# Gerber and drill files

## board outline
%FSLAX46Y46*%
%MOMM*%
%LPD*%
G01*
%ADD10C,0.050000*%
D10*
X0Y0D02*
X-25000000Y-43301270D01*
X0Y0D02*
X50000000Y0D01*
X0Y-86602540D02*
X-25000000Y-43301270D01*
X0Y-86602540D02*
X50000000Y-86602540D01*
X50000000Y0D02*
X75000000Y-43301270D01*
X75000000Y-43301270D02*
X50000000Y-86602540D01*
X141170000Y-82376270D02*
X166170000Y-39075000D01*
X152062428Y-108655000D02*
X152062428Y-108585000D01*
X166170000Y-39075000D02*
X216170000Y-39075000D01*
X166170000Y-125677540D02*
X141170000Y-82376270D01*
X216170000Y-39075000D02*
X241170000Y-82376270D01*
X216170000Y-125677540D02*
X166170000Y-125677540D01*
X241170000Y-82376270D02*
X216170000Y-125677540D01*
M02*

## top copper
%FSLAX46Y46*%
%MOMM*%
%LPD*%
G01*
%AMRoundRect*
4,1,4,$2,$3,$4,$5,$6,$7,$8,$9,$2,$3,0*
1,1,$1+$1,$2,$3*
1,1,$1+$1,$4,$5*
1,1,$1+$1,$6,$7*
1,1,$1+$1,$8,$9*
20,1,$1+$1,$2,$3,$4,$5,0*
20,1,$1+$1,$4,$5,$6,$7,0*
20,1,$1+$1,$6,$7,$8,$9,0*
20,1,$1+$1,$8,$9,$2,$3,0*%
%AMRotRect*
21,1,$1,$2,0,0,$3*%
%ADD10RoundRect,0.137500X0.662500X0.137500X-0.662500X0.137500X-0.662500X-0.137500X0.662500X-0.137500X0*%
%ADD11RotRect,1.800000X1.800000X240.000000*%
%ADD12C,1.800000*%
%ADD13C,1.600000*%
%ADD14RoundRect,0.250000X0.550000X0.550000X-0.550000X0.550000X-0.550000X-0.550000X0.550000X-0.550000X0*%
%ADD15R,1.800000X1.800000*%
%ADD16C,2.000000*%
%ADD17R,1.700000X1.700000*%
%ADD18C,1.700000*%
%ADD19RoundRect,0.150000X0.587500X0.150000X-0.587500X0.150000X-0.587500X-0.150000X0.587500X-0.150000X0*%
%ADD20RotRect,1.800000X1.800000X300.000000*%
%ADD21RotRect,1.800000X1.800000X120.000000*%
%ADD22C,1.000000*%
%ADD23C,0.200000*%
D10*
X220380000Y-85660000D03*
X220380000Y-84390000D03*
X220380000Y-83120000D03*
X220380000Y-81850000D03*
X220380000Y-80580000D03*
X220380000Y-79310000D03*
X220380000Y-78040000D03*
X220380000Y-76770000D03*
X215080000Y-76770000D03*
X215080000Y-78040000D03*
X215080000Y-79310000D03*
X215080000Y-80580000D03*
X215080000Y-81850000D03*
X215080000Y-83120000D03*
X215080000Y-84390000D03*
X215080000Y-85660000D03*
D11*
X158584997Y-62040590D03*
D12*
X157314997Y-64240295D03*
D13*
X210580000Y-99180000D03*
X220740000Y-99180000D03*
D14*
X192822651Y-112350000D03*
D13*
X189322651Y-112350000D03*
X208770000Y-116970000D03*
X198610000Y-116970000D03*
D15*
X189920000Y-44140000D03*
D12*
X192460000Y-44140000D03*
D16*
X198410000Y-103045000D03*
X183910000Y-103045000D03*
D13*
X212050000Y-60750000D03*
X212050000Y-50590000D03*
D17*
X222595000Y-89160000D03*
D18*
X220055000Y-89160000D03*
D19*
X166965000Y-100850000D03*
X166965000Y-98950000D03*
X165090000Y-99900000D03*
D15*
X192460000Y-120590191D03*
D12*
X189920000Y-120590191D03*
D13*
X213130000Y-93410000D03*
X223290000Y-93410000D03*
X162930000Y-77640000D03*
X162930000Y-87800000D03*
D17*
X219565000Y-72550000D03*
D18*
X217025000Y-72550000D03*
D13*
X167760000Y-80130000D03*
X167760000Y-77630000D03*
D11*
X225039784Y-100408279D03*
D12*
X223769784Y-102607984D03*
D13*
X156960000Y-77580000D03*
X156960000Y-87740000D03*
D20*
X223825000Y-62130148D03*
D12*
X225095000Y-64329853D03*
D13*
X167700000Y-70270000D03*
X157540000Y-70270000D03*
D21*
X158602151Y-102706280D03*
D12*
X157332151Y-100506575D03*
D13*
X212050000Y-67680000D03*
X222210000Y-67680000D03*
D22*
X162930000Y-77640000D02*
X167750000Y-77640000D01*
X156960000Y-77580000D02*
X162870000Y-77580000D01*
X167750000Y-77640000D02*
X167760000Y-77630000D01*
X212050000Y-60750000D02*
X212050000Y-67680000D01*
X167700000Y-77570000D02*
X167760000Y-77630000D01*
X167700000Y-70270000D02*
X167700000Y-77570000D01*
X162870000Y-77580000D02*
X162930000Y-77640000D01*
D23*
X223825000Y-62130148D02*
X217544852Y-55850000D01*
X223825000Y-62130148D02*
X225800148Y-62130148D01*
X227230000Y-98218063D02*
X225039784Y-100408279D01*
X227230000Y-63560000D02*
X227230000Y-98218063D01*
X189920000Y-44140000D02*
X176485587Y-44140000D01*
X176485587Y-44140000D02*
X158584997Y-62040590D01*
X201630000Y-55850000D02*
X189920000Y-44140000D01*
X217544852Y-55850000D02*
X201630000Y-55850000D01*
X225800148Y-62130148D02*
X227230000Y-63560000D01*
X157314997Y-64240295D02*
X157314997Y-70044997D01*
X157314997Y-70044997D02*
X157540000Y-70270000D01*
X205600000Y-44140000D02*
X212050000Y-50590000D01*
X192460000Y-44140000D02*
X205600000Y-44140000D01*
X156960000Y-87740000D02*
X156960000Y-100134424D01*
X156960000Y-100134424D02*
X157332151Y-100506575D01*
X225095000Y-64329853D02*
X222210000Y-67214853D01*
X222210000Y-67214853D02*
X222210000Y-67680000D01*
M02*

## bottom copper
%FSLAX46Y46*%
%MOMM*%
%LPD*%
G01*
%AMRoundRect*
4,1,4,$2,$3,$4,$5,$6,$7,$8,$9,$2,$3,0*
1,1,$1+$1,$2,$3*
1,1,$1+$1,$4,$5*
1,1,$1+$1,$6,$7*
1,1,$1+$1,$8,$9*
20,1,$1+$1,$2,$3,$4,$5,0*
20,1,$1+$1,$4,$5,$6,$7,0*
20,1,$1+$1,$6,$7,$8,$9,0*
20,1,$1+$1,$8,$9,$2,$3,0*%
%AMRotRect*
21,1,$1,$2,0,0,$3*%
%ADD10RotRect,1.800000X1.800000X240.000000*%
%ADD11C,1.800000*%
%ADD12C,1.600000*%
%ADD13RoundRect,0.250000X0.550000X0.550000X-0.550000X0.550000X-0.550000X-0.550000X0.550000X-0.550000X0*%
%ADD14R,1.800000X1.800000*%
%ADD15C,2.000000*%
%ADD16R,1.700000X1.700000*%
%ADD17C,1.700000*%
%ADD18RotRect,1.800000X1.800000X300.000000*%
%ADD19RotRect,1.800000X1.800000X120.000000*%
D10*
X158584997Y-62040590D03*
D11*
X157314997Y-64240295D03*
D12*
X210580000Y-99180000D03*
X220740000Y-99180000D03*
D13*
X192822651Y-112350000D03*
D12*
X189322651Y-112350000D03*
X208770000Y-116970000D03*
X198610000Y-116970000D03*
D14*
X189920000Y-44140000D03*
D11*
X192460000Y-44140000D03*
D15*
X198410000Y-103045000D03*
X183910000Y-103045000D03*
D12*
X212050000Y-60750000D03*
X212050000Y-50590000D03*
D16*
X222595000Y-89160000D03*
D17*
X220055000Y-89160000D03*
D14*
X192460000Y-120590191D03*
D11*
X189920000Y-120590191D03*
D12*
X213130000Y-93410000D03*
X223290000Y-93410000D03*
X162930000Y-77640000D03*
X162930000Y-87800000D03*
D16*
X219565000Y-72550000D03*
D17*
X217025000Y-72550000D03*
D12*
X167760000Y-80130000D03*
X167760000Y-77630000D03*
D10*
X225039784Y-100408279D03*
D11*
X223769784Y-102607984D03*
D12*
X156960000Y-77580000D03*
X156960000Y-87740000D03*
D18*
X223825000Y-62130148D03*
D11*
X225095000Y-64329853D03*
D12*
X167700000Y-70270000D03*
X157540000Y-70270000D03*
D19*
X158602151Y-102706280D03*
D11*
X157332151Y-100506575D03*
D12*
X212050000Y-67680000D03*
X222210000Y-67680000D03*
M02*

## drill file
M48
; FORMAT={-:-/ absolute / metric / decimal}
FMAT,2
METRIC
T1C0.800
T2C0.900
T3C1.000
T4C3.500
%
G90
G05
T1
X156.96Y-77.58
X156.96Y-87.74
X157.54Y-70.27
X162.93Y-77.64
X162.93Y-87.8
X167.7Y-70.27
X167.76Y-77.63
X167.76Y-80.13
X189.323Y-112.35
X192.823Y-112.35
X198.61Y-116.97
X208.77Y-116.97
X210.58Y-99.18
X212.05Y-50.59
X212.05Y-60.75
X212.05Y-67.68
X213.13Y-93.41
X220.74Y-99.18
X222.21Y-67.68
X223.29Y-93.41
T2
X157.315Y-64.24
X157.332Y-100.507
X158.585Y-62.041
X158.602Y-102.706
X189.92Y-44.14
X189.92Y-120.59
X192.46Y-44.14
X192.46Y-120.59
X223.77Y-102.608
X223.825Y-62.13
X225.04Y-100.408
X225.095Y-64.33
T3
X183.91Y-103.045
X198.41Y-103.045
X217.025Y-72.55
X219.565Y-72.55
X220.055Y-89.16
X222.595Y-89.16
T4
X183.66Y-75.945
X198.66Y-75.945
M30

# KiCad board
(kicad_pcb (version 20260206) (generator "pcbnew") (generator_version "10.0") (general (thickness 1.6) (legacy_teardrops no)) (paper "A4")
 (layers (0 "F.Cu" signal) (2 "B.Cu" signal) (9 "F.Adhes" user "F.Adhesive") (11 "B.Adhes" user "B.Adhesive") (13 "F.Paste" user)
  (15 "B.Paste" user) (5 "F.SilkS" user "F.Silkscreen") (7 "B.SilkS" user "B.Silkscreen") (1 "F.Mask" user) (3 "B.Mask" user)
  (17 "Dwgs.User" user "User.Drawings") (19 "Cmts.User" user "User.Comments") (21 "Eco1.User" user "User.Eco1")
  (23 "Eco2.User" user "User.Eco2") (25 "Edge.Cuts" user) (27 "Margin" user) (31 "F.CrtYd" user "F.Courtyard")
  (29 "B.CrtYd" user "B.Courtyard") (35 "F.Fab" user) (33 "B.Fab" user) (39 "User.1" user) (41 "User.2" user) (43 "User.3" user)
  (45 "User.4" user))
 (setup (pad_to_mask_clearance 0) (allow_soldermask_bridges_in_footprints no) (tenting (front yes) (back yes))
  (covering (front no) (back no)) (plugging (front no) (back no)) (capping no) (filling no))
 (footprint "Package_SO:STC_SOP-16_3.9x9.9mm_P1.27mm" (layer "F.Cu") (at 217.73 81.215 180)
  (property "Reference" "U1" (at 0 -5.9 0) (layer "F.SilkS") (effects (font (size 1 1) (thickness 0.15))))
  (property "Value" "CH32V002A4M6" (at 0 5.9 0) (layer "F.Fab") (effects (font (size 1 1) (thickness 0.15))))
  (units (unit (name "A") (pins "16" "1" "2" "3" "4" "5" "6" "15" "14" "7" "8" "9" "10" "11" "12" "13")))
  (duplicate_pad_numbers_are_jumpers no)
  (pad "1" smd roundrect (at -2.65 -4.445 180) (size 1.6 0.55) (layers "F.Cu" "F.Mask" "F.Paste") (roundrect_rratio 0.25)
   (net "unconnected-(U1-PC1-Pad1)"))
  (pad "2" smd roundrect (at -2.65 -3.175 180) (size 1.6 0.55) (layers "F.Cu" "F.Mask" "F.Paste") (roundrect_rratio 0.25)
   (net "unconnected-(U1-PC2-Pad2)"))
  (pad "3" smd roundrect (at -2.65 -1.905 180) (size 1.6 0.55) (layers "F.Cu" "F.Mask" "F.Paste") (roundrect_rratio 0.25) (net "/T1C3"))
  (pad "4" smd roundrect (at -2.65 -0.635 180) (size 1.6 0.55) (layers "F.Cu" "F.Mask" "F.Paste") (roundrect_rratio 0.25)
   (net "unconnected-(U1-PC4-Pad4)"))
  (pad "5" smd roundrect (at -2.65 0.635 180) (size 1.6 0.55) (layers "F.Cu" "F.Mask" "F.Paste") (roundrect_rratio 0.25)
   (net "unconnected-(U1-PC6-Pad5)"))
  (pad "6" smd roundrect (at -2.65 1.905 180) (size 1.6 0.55) (layers "F.Cu" "F.Mask" "F.Paste") (roundrect_rratio 0.25)
   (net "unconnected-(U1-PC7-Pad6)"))
  (pad "7" smd roundrect (at -2.65 3.175 180) (size 1.6 0.55) (layers "F.Cu" "F.Mask" "F.Paste") (roundrect_rratio 0.25) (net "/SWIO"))
  (pad "8" smd roundrect (at -2.65 4.445 180) (size 1.6 0.55) (layers "F.Cu" "F.Mask" "F.Paste") (roundrect_rratio 0.25)
   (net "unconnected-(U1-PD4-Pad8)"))
  (pad "9" smd roundrect (at 2.65 4.445 180) (size 1.6 0.55) (layers "F.Cu" "F.Mask" "F.Paste") (roundrect_rratio 0.25)
   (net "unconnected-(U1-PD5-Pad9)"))
  (pad "10" smd roundrect (at 2.65 3.175 180) (size 1.6 0.55) (layers "F.Cu" "F.Mask" "F.Paste") (roundrect_rratio 0.25)
   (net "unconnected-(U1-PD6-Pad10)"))
  (pad "11" smd roundrect (at 2.65 1.905 180) (size 1.6 0.55) (layers "F.Cu" "F.Mask" "F.Paste") (roundrect_rratio 0.25)
   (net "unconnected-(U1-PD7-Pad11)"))
  (pad "12" smd roundrect (at 2.65 0.635 180) (size 1.6 0.55) (layers "F.Cu" "F.Mask" "F.Paste") (roundrect_rratio 0.25)
   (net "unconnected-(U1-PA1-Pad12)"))
  (pad "13" smd roundrect (at 2.65 -0.635 180) (size 1.6 0.55) (layers "F.Cu" "F.Mask" "F.Paste") (roundrect_rratio 0.25)
   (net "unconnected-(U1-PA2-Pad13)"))
  (pad "14" smd roundrect (at 2.65 -1.905 180) (size 1.6 0.55) (layers "F.Cu" "F.Mask" "F.Paste") (roundrect_rratio 0.25) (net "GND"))
  (pad "15" smd roundrect (at 2.65 -3.175 180) (size 1.6 0.55) (layers "F.Cu" "F.Mask" "F.Paste") (roundrect_rratio 0.25) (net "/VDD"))
  (pad "16" smd roundrect (at 2.65 -4.445 180) (size 1.6 0.55) (layers "F.Cu" "F.Mask" "F.Paste") (roundrect_rratio 0.25)
   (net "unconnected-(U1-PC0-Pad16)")))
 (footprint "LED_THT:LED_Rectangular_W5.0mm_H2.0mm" (layer "F.Cu") (at 158.584997 62.04059 -120)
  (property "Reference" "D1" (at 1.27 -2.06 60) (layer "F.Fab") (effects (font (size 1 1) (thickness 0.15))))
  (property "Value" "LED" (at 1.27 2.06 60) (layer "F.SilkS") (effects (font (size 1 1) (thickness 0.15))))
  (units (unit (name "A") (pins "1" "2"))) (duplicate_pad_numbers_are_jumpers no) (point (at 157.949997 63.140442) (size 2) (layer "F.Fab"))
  (pad "1" thru_hole rect (at 0 0 240) (size 1.8 1.8) (drill 0.9) (layers "*.Cu" "*.Mask") (remove_unused_layers no) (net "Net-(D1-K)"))
  (pad "2" thru_hole circle (at 2.54 0 240) (size 1.8 1.8) (drill 0.9) (layers "*.Cu" "*.Mask") (remove_unused_layers no) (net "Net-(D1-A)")))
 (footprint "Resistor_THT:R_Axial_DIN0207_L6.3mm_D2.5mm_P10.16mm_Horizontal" (layer "F.Cu") (at 210.58 99.18)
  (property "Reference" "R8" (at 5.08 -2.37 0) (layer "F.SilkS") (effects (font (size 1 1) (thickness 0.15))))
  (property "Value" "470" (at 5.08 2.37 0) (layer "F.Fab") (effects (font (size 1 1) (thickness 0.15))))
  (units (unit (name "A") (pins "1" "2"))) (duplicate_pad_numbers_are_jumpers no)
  (pad "1" thru_hole circle (at 0 0) (size 1.6 1.6) (drill 0.8) (layers "*.Cu" "*.Mask") (remove_unused_layers no) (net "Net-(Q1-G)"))
  (pad "2" thru_hole circle (at 10.16 0) (size 1.6 1.6) (drill 0.8) (layers "*.Cu" "*.Mask") (remove_unused_layers no) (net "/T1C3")))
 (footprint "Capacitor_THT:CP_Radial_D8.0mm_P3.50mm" (layer "F.Cu") (at 192.822651 112.35 180)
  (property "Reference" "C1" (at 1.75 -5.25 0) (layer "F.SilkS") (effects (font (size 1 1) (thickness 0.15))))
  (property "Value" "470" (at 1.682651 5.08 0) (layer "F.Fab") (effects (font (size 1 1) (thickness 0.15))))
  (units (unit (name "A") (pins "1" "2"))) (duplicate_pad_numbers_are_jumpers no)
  (pad "1" thru_hole roundrect (at 0 0 180) (size 1.6 1.6) (drill 0.8) (layers "*.Cu" "*.Mask") (remove_unused_layers no)
   (roundrect_rratio 0.15625) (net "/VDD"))
  (pad "2" thru_hole circle (at 3.5 0 180) (size 1.6 1.6) (drill 0.8) (layers "*.Cu" "*.Mask") (remove_unused_layers no) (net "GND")))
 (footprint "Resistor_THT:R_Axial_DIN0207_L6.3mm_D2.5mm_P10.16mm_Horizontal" (layer "F.Cu") (at 208.77 116.97 180)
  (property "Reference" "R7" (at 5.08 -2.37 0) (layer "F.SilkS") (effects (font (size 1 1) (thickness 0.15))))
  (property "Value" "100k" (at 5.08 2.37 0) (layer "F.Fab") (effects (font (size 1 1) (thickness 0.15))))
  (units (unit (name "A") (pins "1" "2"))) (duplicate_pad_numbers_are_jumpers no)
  (pad "1" thru_hole circle (at 0 0 180) (size 1.6 1.6) (drill 0.8) (layers "*.Cu" "*.Mask") (remove_unused_layers no) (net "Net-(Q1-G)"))
  (pad "2" thru_hole circle (at 10.16 0 180) (size 1.6 1.6) (drill 0.8) (layers "*.Cu" "*.Mask") (remove_unused_layers no) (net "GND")))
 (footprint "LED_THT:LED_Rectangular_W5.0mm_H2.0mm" (layer "F.Cu") (at 189.92 44.14)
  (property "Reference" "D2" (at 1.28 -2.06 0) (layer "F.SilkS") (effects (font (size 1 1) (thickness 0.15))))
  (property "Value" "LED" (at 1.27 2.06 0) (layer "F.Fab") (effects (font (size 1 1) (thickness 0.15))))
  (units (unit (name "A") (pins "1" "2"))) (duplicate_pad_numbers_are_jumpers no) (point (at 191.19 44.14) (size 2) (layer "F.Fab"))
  (pad "1" thru_hole rect (at 0 0) (size 1.8 1.8) (drill 0.9) (layers "*.Cu" "*.Mask") (remove_unused_layers no) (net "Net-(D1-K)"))
  (pad "2" thru_hole circle (at 2.54 0) (size 1.8 1.8) (drill 0.9) (layers "*.Cu" "*.Mask") (remove_unused_layers no) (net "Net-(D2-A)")))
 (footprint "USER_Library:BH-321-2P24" (layer "F.Cu") (at 191.16 75.945 -90)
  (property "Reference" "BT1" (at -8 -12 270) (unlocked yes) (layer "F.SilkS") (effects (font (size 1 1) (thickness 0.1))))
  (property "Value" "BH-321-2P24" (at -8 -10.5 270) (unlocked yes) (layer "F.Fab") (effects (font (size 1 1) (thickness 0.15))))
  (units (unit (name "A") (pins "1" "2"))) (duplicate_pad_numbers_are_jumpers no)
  (pad "" np_thru_hole circle (at 0 -7.5 270) (size 3.5 3.5) (drill 3.5) (layers "*.Cu" "*.Mask") (thermal_bridge_angle 90))
  (pad "" np_thru_hole circle (at 0 7.5 270) (size 3.5 3.5) (drill 3.5) (layers "*.Cu" "*.Mask") (thermal_bridge_angle 90))
  (pad "1" thru_hole circle (at 27.1 -7.25 270) (size 2 2) (drill 1) (layers "*.Cu" "*.Mask") (remove_unused_layers no) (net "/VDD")
   (thermal_bridge_angle 90))
  (pad "2" thru_hole circle (at 27.1 7.25 270) (size 2 2) (drill 1) (layers "*.Cu" "*.Mask") (remove_unused_layers no) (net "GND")
   (thermal_bridge_angle 90)))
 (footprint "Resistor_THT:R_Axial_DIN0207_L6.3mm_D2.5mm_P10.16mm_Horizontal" (layer "F.Cu") (at 212.05 60.75 90)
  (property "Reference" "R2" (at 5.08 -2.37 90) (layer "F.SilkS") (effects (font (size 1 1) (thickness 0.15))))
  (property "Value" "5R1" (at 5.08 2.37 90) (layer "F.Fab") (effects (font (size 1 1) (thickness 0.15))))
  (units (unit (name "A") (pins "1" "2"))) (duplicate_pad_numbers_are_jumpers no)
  (pad "1" thru_hole circle (at 0 0 90) (size 1.6 1.6) (drill 0.8) (layers "*.Cu" "*.Mask") (remove_unused_layers no) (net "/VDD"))
  (pad "2" thru_hole circle (at 10.16 0 90) (size 1.6 1.6) (drill 0.8) (layers "*.Cu" "*.Mask") (remove_unused_layers no) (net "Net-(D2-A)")))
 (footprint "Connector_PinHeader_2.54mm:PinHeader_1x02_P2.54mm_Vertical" (layer "F.Cu") (at 222.595 89.16 -90)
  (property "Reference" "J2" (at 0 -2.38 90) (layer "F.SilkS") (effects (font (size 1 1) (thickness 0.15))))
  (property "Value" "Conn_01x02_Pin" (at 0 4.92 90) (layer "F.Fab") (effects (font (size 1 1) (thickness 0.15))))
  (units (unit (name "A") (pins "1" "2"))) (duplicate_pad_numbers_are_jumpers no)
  (pad "1" thru_hole rect (at 0 0 270) (size 1.7 1.7) (drill 1) (layers "*.Cu" "*.Mask") (remove_unused_layers no) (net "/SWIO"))
  (pad "2" thru_hole circle (at 0 2.54 270) (size 1.7 1.7) (drill 1) (layers "*.Cu" "*.Mask") (remove_unused_layers no) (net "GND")))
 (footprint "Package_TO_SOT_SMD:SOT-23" (layer "F.Cu") (at 166.0275 99.9 180)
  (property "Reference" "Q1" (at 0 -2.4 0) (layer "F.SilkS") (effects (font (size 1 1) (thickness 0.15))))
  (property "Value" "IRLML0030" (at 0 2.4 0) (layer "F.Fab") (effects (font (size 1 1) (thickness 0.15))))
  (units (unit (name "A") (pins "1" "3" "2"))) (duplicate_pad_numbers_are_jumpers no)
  (pad "1" smd roundrect (at -0.9375 -0.95 180) (size 1.475 0.6) (layers "F.Cu" "F.Mask" "F.Paste") (roundrect_rratio 0.25)
   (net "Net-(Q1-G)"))
  (pad "2" smd roundrect (at -0.9375 0.95 180) (size 1.475 0.6) (layers "F.Cu" "F.Mask" "F.Paste") (roundrect_rratio 0.25) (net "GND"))
  (pad "3" smd roundrect (at 0.9375 0 180) (size 1.475 0.6) (layers "F.Cu" "F.Mask" "F.Paste") (roundrect_rratio 0.25) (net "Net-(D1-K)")))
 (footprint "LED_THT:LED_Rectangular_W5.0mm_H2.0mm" (layer "F.Cu") (at 192.46 120.590191 180)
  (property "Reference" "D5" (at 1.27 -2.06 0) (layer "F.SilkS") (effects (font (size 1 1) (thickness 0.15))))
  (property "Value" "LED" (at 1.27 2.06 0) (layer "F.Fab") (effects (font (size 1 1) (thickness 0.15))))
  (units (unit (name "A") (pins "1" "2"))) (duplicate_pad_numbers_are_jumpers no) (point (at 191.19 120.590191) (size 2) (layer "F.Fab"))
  (pad "1" thru_hole rect (at 0 0 180) (size 1.8 1.8) (drill 0.9) (layers "*.Cu" "*.Mask") (remove_unused_layers no) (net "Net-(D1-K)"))
  (pad "2" thru_hole circle (at 2.54 0 180) (size 1.8 1.8) (drill 0.9) (layers "*.Cu" "*.Mask") (remove_unused_layers no) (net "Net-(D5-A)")))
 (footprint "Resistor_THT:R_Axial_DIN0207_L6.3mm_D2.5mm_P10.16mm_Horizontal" (layer "F.Cu") (at 213.13 93.41)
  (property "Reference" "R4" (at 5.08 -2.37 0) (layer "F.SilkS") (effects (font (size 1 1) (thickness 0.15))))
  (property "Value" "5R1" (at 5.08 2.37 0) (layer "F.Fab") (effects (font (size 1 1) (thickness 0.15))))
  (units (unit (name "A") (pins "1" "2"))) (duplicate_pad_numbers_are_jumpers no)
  (pad "1" thru_hole circle (at 0 0) (size 1.6 1.6) (drill 0.8) (layers "*.Cu" "*.Mask") (remove_unused_layers no) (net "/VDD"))
  (pad "2" thru_hole circle (at 10.16 0) (size 1.6 1.6) (drill 0.8) (layers "*.Cu" "*.Mask") (remove_unused_layers no) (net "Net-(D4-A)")))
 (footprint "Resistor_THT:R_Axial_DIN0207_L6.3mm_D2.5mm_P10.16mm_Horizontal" (layer "F.Cu") (at 162.93 77.64 -90)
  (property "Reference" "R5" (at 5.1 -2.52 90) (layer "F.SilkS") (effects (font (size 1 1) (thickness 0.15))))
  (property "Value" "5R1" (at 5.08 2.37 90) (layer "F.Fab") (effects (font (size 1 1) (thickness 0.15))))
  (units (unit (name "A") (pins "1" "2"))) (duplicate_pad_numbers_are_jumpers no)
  (pad "1" thru_hole circle (at 0 0 270) (size 1.6 1.6) (drill 0.8) (layers "*.Cu" "*.Mask") (remove_unused_layers no) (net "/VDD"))
  (pad "2" thru_hole circle (at 10.16 0 270) (size 1.6 1.6) (drill 0.8) (layers "*.Cu" "*.Mask") (remove_unused_layers no)
   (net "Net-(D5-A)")))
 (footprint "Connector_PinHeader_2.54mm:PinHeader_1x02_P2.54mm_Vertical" (layer "F.Cu") (at 219.565 72.55 -90)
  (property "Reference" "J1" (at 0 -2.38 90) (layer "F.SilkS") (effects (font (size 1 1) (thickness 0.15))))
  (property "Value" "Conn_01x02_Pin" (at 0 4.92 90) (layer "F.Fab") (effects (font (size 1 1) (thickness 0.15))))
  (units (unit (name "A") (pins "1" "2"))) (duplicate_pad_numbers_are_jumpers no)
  (pad "1" thru_hole rect (at 0 0 270) (size 1.7 1.7) (drill 1) (layers "*.Cu" "*.Mask") (remove_unused_layers no) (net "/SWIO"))
  (pad "2" thru_hole circle (at 0 2.54 270) (size 1.7 1.7) (drill 1) (layers "*.Cu" "*.Mask") (remove_unused_layers no) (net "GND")))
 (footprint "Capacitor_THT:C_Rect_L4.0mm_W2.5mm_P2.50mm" (layer "F.Cu") (at 167.76 80.13 90)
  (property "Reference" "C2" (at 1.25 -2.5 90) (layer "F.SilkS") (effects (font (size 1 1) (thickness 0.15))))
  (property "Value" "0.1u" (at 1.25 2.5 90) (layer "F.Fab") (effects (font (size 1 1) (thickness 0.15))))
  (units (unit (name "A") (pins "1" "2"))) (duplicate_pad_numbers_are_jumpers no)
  (pad "1" thru_hole circle (at 0 0 90) (size 1.6 1.6) (drill 0.8) (layers "*.Cu" "*.Mask") (remove_unused_layers no) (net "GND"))
  (pad "2" thru_hole circle (at 2.5 0 90) (size 1.6 1.6) (drill 0.8) (layers "*.Cu" "*.Mask") (remove_unused_layers no) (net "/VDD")))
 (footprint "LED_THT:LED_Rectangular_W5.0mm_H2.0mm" (layer "F.Cu") (at 225.039784 100.408279 -120)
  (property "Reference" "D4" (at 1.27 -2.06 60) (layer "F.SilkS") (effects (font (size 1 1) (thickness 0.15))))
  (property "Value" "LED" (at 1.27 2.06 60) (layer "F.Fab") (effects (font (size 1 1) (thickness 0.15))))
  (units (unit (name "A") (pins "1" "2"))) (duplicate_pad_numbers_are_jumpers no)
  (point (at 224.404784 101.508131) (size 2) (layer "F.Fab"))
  (pad "1" thru_hole rect (at 0 0 240) (size 1.8 1.8) (drill 0.9) (layers "*.Cu" "*.Mask") (remove_unused_layers no) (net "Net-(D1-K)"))
  (pad "2" thru_hole circle (at 2.54 0 240) (size 1.8 1.8) (drill 0.9) (layers "*.Cu" "*.Mask") (remove_unused_layers no) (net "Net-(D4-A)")))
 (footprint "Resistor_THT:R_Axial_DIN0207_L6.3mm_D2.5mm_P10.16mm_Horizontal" (layer "F.Cu") (at 156.96 77.58 -90)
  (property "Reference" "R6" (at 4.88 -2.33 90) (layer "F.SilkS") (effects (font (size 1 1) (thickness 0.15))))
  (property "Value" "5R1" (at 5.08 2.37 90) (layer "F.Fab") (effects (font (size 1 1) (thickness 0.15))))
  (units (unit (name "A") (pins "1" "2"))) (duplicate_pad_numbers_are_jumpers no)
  (pad "1" thru_hole circle (at 0 0 270) (size 1.6 1.6) (drill 0.8) (layers "*.Cu" "*.Mask") (remove_unused_layers no) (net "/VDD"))
  (pad "2" thru_hole circle (at 10.16 0 270) (size 1.6 1.6) (drill 0.8) (layers "*.Cu" "*.Mask") (remove_unused_layers no)
   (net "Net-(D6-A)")))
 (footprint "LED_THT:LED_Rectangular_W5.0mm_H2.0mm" (layer "F.Cu") (at 223.825 62.130148 -60)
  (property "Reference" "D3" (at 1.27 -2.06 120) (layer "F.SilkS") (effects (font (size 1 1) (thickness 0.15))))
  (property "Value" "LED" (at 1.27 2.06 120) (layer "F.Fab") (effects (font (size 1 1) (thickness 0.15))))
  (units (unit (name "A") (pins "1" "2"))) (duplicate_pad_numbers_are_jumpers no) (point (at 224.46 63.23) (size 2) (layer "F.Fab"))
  (pad "1" thru_hole rect (at 0 0 300) (size 1.8 1.8) (drill 0.9) (layers "*.Cu" "*.Mask") (remove_unused_layers no) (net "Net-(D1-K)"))
  (pad "2" thru_hole circle (at 2.54 0 300) (size 1.8 1.8) (drill 0.9) (layers "*.Cu" "*.Mask") (remove_unused_layers no) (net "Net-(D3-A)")))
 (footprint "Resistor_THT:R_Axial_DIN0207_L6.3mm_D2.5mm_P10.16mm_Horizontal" (layer "F.Cu") (at 167.7 70.27 180)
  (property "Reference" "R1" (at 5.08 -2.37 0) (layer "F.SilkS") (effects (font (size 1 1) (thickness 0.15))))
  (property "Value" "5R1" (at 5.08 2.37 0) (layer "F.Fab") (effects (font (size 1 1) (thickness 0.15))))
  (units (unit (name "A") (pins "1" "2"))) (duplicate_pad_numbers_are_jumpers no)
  (pad "1" thru_hole circle (at 0 0 180) (size 1.6 1.6) (drill 0.8) (layers "*.Cu" "*.Mask") (remove_unused_layers no) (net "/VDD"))
  (pad "2" thru_hole circle (at 10.16 0 180) (size 1.6 1.6) (drill 0.8) (layers "*.Cu" "*.Mask") (remove_unused_layers no)
   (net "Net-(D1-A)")))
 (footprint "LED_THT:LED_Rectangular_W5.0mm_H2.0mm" (layer "F.Cu") (at 158.602151 102.70628 120)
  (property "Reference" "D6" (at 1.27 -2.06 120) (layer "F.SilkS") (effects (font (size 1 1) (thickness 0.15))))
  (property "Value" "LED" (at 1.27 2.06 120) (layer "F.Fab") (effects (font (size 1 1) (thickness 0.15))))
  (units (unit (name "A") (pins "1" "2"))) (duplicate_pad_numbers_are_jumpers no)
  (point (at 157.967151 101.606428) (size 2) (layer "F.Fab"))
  (pad "1" thru_hole rect (at 0 0 120) (size 1.8 1.8) (drill 0.9) (layers "*.Cu" "*.Mask") (remove_unused_layers no) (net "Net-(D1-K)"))
  (pad "2" thru_hole circle (at 2.54 0 120) (size 1.8 1.8) (drill 0.9) (layers "*.Cu" "*.Mask") (remove_unused_layers no) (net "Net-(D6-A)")))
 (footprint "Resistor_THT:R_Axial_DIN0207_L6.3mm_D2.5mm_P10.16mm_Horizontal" (layer "F.Cu") (at 212.05 67.68)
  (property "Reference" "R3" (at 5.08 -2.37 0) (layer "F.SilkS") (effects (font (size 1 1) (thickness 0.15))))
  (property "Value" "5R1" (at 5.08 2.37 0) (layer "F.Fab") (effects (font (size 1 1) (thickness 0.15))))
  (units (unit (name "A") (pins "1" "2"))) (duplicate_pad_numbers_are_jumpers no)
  (pad "1" thru_hole circle (at 0 0) (size 1.6 1.6) (drill 0.8) (layers "*.Cu" "*.Mask") (remove_unused_layers no) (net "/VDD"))
  (pad "2" thru_hole circle (at 10.16 0) (size 1.6 1.6) (drill 0.8) (layers "*.Cu" "*.Mask") (remove_unused_layers no) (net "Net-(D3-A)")))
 (gr_line (start 0 0) (end -25 43.30127) (stroke (width 0.05) (type solid)) (locked yes) (layer "Edge.Cuts"))
 (gr_line (start 0 0) (end 50 0) (stroke (width 0.05) (type solid)) (locked yes) (layer "Edge.Cuts"))
 (gr_line (start 0 86.60254) (end -25 43.30127) (stroke (width 0.05) (type solid)) (locked yes) (layer "Edge.Cuts"))
 (gr_line (start 0 86.60254) (end 50 86.60254) (stroke (width 0.05) (type solid)) (locked yes) (layer "Edge.Cuts"))
 (gr_line (start 50 0) (end 75 43.30127) (stroke (width 0.05) (type solid)) (locked yes) (layer "Edge.Cuts"))
 (gr_line (start 75 43.30127) (end 50 86.60254) (stroke (width 0.05) (type solid)) (locked yes) (layer "Edge.Cuts"))
 (gr_line (start 141.17 82.37627) (end 166.17 39.075) (stroke (width 0.05) (type default)) (layer "Edge.Cuts"))
 (gr_line (start 152.062428 108.655) (end 152.062428 108.585) (stroke (width 0.05) (type default)) (layer "Edge.Cuts"))
 (gr_line (start 166.17 39.075) (end 216.17 39.075) (stroke (width 0.05) (type solid)) (layer "Edge.Cuts"))
 (gr_line (start 166.17 125.67754) (end 141.17 82.37627) (stroke (width 0.05) (type solid)) (layer "Edge.Cuts"))
 (gr_line (start 216.17 39.075) (end 241.17 82.37627) (stroke (width 0.05) (type solid)) (layer "Edge.Cuts"))
 (gr_line (start 216.17 125.67754) (end 166.17 125.67754) (stroke (width 0.05) (type solid)) (layer "Edge.Cuts"))
 (gr_line (start 241.17 82.37627) (end 216.17 125.67754) (stroke (width 0.05) (type solid)) (layer "Edge.Cuts"))
 (segment (start 162.93 77.64) (end 167.75 77.64) (width 1) (layer "F.Cu") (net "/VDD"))
 (segment (start 156.96 77.58) (end 162.87 77.58) (width 1) (layer "F.Cu") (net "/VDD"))
 (segment (start 167.75 77.64) (end 167.76 77.63) (width 1) (layer "F.Cu") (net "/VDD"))
 (segment (start 212.05 60.75) (end 212.05 67.68) (width 1) (layer "F.Cu") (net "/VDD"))
 (segment (start 167.7 77.57) (end 167.76 77.63) (width 1) (layer "F.Cu") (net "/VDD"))
 (segment (start 167.7 70.27) (end 167.7 77.57) (width 1) (layer "F.Cu") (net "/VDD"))
 (segment (start 162.87 77.58) (end 162.93 77.64) (width 1) (layer "F.Cu") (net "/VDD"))
 (segment (start 223.825 62.130148) (end 217.544852 55.85) (width 0.2) (layer "F.Cu") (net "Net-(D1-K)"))
 (segment (start 223.825 62.130148) (end 225.800148 62.130148) (width 0.2) (layer "F.Cu") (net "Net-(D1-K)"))
 (segment (start 227.23 98.218063) (end 225.039784 100.408279) (width 0.2) (layer "F.Cu") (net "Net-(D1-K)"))
 (segment (start 227.23 63.56) (end 227.23 98.218063) (width 0.2) (layer "F.Cu") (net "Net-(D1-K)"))
 (segment (start 189.92 44.14) (end 176.485587 44.14) (width 0.2) (layer "F.Cu") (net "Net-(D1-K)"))
 (segment (start 176.485587 44.14) (end 158.584997 62.04059) (width 0.2) (layer "F.Cu") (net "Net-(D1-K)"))
 (segment (start 201.63 55.85) (end 189.92 44.14) (width 0.2) (layer "F.Cu") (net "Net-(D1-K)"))
 (segment (start 217.544852 55.85) (end 201.63 55.85) (width 0.2) (layer "F.Cu") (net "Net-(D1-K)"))
 (segment (start 225.800148 62.130148) (end 227.23 63.56) (width 0.2) (layer "F.Cu") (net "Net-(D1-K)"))
 (segment (start 157.314997 64.240295) (end 157.314997 70.044997) (width 0.2) (layer "F.Cu") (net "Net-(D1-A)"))
 (segment (start 157.314997 70.044997) (end 157.54 70.27) (width 0.2) (layer "F.Cu") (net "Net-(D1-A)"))
 (segment (start 205.6 44.14) (end 212.05 50.59) (width 0.2) (layer "F.Cu") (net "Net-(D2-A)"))
 (segment (start 192.46 44.14) (end 205.6 44.14) (width 0.2) (layer "F.Cu") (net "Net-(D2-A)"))
 (segment (start 156.96 87.74) (end 156.96 100.134424) (width 0.2) (layer "F.Cu") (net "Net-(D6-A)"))
 (segment (start 156.96 100.134424) (end 157.332151 100.506575) (width 0.2) (layer "F.Cu") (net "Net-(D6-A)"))
 (segment (start 225.095 64.329853) (end 222.21 67.214853) (width 0.2) (layer "F.Cu") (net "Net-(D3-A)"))
 (segment (start 222.21 67.214853) (end 222.21 67.68) (width 0.2) (layer "F.Cu") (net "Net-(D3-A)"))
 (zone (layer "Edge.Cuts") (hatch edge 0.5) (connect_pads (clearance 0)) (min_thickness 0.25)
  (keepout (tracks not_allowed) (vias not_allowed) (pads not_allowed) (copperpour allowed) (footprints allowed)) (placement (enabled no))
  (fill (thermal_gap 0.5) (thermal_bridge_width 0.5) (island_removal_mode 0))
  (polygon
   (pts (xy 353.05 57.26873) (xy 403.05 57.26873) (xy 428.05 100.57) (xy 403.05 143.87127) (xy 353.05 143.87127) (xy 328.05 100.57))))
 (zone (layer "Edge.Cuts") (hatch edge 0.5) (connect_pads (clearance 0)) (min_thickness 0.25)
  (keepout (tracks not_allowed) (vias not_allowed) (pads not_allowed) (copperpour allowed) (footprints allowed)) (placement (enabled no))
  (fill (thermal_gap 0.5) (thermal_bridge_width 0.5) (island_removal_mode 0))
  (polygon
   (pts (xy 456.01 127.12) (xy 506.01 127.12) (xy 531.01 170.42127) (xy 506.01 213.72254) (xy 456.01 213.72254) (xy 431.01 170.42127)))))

